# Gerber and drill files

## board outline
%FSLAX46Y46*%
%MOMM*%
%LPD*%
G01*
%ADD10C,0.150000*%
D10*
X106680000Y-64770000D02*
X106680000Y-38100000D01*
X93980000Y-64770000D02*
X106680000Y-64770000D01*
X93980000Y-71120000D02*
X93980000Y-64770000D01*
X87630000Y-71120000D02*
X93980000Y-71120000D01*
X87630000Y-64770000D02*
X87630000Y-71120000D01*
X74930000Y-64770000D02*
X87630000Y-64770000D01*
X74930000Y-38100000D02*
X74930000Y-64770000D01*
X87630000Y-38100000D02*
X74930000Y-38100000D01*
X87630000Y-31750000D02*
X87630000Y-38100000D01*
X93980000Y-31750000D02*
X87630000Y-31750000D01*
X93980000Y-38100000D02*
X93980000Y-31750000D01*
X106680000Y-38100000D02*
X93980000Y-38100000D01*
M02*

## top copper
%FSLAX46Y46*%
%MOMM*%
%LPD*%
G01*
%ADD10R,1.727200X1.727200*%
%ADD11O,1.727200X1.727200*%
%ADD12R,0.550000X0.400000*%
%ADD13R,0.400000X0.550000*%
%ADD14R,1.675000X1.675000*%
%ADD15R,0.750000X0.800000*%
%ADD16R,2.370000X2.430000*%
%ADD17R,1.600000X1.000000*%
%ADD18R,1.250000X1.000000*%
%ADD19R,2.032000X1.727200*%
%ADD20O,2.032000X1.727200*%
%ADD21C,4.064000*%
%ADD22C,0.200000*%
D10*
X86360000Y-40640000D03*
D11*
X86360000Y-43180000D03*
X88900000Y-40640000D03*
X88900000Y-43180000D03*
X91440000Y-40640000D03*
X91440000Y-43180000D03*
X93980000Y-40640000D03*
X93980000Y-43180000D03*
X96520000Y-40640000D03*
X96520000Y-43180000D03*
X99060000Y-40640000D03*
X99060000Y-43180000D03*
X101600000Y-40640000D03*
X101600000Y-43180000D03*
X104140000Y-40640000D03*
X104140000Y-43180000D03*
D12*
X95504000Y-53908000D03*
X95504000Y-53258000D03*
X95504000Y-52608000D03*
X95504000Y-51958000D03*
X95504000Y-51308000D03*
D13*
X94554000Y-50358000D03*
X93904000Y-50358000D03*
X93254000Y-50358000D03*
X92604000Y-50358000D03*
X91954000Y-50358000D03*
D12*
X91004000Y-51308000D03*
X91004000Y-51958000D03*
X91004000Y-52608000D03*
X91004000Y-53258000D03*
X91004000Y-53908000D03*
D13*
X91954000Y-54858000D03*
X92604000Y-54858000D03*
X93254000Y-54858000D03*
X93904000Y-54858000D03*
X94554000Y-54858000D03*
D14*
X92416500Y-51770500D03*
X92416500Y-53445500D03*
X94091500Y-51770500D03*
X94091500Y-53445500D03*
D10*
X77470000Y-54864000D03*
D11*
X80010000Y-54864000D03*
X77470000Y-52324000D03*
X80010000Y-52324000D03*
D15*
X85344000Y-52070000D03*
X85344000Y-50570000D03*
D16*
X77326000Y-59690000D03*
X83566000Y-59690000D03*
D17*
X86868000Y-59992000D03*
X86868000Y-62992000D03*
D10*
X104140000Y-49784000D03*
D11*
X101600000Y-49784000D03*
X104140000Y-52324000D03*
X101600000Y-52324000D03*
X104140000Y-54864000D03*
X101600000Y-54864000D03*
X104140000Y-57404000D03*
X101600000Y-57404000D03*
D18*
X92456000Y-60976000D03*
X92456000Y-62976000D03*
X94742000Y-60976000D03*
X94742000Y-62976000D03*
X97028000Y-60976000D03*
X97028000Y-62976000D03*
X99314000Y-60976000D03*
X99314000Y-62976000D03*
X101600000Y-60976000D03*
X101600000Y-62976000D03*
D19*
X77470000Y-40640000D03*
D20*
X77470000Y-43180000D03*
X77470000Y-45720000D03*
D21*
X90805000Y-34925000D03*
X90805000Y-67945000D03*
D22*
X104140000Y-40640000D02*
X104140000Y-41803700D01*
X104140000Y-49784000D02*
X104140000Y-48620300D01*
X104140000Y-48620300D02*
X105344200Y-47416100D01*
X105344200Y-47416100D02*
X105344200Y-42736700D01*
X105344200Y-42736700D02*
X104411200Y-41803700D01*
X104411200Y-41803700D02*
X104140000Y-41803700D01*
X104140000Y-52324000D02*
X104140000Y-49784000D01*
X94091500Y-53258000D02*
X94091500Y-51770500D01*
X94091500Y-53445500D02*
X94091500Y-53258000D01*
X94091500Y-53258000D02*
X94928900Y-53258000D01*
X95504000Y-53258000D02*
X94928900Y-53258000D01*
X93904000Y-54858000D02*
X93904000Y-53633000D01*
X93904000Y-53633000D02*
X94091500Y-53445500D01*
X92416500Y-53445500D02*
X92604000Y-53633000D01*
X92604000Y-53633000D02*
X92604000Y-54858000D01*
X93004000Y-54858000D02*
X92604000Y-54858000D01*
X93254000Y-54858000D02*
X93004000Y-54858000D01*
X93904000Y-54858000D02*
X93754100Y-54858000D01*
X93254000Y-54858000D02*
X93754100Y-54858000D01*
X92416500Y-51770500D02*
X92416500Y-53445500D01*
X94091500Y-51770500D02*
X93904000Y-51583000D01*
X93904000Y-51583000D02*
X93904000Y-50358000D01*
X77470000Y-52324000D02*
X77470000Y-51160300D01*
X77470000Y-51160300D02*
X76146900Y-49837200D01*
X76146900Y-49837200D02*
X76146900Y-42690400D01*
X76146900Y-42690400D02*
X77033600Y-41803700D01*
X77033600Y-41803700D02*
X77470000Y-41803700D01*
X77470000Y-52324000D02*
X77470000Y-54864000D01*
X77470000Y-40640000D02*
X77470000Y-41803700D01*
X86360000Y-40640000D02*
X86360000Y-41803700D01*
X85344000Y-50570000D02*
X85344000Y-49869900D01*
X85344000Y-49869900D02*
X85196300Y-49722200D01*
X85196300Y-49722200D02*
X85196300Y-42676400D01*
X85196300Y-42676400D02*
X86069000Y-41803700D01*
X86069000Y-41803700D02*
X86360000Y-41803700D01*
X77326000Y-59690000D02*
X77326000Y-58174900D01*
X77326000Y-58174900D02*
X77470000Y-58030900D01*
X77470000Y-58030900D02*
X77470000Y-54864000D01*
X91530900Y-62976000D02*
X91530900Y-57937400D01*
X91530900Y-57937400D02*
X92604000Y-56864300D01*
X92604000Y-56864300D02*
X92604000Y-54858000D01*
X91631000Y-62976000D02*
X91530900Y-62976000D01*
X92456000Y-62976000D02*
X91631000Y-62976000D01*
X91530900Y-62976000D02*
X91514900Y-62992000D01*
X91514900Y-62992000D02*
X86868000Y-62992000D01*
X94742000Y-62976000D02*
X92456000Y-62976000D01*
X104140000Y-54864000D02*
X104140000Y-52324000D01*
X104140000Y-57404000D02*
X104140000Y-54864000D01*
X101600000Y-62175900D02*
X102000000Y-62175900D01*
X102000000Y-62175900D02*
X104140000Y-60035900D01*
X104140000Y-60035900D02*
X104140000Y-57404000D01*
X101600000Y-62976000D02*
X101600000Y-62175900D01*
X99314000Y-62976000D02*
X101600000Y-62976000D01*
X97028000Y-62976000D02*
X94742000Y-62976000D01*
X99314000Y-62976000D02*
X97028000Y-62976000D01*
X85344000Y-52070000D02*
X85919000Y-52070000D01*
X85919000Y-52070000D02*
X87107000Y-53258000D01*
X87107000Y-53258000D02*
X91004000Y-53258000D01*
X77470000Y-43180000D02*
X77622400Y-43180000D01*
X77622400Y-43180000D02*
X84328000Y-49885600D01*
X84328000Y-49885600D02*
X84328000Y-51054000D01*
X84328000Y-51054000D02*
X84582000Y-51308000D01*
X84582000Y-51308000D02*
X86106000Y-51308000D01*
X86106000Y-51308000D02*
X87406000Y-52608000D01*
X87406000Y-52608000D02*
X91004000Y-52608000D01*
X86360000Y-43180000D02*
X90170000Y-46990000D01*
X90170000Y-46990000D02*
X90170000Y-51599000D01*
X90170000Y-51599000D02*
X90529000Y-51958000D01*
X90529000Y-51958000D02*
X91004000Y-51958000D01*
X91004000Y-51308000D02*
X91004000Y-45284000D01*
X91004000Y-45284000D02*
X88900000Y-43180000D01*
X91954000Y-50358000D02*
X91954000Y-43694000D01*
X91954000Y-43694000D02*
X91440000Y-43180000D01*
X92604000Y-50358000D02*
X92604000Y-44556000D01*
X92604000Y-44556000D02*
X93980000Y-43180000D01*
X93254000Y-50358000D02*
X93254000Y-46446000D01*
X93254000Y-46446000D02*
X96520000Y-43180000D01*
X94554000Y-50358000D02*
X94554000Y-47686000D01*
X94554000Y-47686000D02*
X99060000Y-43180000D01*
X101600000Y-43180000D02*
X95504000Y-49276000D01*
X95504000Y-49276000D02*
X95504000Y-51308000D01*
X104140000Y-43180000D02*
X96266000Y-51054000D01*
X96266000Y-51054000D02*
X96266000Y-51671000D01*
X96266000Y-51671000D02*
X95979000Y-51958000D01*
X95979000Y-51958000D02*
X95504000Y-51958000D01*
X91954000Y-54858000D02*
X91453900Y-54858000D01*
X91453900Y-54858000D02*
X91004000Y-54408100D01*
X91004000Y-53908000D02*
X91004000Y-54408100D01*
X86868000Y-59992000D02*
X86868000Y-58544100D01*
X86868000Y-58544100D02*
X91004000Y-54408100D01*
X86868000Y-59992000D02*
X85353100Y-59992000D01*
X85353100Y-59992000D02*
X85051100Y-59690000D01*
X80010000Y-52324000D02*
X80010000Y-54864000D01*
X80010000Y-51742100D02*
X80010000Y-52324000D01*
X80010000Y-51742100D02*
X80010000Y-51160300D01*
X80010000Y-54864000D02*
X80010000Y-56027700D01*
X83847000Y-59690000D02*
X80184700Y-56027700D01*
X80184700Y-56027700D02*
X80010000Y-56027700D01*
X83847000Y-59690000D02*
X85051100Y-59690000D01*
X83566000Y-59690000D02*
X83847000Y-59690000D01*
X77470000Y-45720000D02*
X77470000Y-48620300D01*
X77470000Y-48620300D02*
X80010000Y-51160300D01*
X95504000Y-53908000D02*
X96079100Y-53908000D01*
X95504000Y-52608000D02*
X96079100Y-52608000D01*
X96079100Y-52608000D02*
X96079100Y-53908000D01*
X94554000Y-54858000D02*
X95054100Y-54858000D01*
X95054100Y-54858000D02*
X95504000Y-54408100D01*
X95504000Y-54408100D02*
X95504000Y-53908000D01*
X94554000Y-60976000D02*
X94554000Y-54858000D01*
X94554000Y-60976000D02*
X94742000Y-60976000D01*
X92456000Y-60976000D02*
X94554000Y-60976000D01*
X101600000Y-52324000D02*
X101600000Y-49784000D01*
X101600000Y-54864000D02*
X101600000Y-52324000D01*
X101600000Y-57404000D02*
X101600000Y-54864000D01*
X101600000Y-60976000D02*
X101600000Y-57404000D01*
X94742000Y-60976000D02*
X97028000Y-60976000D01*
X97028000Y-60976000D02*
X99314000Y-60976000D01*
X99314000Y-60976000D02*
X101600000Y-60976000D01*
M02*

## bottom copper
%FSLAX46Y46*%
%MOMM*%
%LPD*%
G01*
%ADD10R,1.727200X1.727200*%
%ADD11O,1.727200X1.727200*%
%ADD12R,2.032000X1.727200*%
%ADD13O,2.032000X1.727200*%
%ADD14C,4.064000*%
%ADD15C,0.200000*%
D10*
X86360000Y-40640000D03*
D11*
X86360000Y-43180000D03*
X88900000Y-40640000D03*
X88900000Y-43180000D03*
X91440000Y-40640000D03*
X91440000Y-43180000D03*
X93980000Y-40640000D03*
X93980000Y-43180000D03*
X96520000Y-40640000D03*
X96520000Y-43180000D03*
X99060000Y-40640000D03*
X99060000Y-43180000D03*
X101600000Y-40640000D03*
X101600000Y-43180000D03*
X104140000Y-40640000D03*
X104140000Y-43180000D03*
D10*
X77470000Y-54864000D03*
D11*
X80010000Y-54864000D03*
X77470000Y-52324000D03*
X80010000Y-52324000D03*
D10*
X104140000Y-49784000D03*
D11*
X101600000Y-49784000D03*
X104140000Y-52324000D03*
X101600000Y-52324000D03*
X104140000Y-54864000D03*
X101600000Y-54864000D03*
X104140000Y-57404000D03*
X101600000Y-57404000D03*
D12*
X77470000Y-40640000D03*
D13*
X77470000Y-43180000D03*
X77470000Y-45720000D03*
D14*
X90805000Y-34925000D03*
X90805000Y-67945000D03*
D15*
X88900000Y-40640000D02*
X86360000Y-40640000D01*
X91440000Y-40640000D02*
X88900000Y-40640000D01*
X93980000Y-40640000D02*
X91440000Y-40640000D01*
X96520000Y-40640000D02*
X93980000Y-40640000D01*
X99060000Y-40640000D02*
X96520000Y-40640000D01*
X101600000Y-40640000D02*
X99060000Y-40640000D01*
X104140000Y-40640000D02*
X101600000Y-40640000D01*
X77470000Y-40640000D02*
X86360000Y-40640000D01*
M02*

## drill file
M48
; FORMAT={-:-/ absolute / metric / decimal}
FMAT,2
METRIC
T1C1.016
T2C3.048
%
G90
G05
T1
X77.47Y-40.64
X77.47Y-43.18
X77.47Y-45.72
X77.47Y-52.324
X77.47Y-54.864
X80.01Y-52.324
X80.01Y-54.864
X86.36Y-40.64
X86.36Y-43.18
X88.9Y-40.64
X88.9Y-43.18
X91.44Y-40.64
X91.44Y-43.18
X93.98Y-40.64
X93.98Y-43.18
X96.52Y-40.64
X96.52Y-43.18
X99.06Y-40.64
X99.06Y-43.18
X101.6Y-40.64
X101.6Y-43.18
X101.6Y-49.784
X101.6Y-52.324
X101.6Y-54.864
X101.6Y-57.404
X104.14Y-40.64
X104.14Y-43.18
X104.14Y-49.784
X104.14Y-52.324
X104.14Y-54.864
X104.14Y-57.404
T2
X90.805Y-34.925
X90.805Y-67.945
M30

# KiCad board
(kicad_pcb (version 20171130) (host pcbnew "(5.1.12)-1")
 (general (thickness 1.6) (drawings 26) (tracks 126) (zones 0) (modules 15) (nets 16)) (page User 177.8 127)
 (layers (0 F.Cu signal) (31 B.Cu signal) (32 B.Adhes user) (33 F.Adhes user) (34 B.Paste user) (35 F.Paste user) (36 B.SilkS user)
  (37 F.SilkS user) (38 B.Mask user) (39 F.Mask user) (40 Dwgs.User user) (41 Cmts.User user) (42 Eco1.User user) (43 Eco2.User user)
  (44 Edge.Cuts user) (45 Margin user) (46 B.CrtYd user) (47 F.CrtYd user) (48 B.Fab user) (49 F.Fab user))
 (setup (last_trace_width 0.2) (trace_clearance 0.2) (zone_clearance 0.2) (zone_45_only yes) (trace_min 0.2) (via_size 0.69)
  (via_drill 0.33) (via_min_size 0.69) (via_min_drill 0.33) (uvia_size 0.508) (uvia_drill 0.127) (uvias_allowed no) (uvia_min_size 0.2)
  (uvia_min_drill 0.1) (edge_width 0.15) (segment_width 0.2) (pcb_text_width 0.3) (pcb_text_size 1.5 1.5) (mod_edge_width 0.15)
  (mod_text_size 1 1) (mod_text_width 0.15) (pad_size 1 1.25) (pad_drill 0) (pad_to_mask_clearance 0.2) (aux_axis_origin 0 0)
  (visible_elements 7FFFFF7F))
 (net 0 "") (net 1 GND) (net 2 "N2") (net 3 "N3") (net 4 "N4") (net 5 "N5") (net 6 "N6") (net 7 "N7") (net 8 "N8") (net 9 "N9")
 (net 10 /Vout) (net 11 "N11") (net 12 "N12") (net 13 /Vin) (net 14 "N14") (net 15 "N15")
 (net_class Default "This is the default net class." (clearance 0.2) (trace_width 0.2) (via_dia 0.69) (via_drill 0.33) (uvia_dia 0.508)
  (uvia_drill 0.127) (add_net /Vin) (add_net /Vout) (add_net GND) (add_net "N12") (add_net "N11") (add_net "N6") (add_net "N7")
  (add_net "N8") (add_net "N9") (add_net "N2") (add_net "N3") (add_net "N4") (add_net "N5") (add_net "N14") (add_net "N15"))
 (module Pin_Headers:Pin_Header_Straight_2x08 (layer B.Cu) (at 86.36 40.64 270)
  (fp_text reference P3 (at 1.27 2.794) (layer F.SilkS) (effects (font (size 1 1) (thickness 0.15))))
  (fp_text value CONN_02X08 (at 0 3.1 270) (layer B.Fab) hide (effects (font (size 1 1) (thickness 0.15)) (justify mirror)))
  (pad 1 thru_hole rect (at 0 0 270) (size 1.7272 1.7272) (drill 1.016) (layers *.Cu *.Mask B.SilkS) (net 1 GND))
  (pad 2 thru_hole oval (at 2.54 0 270) (size 1.7272 1.7272) (drill 1.016) (layers *.Cu *.Mask B.SilkS) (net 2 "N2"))
  (pad 3 thru_hole oval (at 0 -2.54 270) (size 1.7272 1.7272) (drill 1.016) (layers *.Cu *.Mask B.SilkS) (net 1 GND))
  (pad 4 thru_hole oval (at 2.54 -2.54 270) (size 1.7272 1.7272) (drill 1.016) (layers *.Cu *.Mask B.SilkS) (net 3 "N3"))
  (pad 5 thru_hole oval (at 0 -5.08 270) (size 1.7272 1.7272) (drill 1.016) (layers *.Cu *.Mask B.SilkS) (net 1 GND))
  (pad 6 thru_hole oval (at 2.54 -5.08 270) (size 1.7272 1.7272) (drill 1.016) (layers *.Cu *.Mask B.SilkS) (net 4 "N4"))
  (pad 7 thru_hole oval (at 0 -7.62 270) (size 1.7272 1.7272) (drill 1.016) (layers *.Cu *.Mask B.SilkS) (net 1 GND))
  (pad 8 thru_hole oval (at 2.54 -7.62 270) (size 1.7272 1.7272) (drill 1.016) (layers *.Cu *.Mask B.SilkS) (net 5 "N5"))
  (pad 9 thru_hole oval (at 0 -10.16 270) (size 1.7272 1.7272) (drill 1.016) (layers *.Cu *.Mask B.SilkS) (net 1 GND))
  (pad 10 thru_hole oval (at 2.54 -10.16 270) (size 1.7272 1.7272) (drill 1.016) (layers *.Cu *.Mask B.SilkS) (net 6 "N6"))
  (pad 11 thru_hole oval (at 0 -12.7 270) (size 1.7272 1.7272) (drill 1.016) (layers *.Cu *.Mask B.SilkS) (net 1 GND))
  (pad 12 thru_hole oval (at 2.54 -12.7 270) (size 1.7272 1.7272) (drill 1.016) (layers *.Cu *.Mask B.SilkS) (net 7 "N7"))
  (pad 13 thru_hole oval (at 0 -15.24 270) (size 1.7272 1.7272) (drill 1.016) (layers *.Cu *.Mask B.SilkS) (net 1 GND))
  (pad 14 thru_hole oval (at 2.54 -15.24 270) (size 1.7272 1.7272) (drill 1.016) (layers *.Cu *.Mask B.SilkS) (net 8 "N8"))
  (pad 15 thru_hole oval (at 0 -17.78 270) (size 1.7272 1.7272) (drill 1.016) (layers *.Cu *.Mask B.SilkS) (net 1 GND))
  (pad 16 thru_hole oval (at 2.54 -17.78 270) (size 1.7272 1.7272) (drill 1.016) (layers *.Cu *.Mask B.SilkS) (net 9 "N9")))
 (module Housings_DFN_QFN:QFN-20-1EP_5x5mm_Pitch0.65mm (layer F.Cu) (at 93.254 52.608 180)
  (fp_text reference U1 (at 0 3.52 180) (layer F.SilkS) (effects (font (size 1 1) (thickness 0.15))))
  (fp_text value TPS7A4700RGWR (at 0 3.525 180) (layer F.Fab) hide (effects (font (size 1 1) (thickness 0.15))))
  (pad 1 smd rect (at -2.25 -1.3 180) (size 0.55 0.4) (layers F.Cu F.Paste F.Mask) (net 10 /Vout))
  (pad 2 smd rect (at -2.25 -0.65 180) (size 0.55 0.4) (layers F.Cu F.Paste F.Mask) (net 1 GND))
  (pad 3 smd rect (at -2.25 0 180) (size 0.55 0.4) (layers F.Cu F.Paste F.Mask) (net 10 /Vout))
  (pad 4 smd rect (at -2.25 0.65 180) (size 0.55 0.4) (layers F.Cu F.Paste F.Mask) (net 9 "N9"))
  (pad 5 smd rect (at -2.25 1.3 180) (size 0.55 0.4) (layers F.Cu F.Paste F.Mask) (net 8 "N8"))
  (pad 6 smd rect (at -1.3 2.25 270) (size 0.55 0.4) (layers F.Cu F.Paste F.Mask) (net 7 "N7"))
  (pad 7 smd rect (at -0.65 2.25 270) (size 0.55 0.4) (layers F.Cu F.Paste F.Mask) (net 1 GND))
  (pad 8 smd rect (at 0 2.25 270) (size 0.55 0.4) (layers F.Cu F.Paste F.Mask) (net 6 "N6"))
  (pad 9 smd rect (at 0.65 2.25 270) (size 0.55 0.4) (layers F.Cu F.Paste F.Mask) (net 5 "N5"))
  (pad 10 smd rect (at 1.3 2.25 270) (size 0.55 0.4) (layers F.Cu F.Paste F.Mask) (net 4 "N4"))
  (pad 11 smd rect (at 2.25 1.3 180) (size 0.55 0.4) (layers F.Cu F.Paste F.Mask) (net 3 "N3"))
  (pad 12 smd rect (at 2.25 0.65 180) (size 0.55 0.4) (layers F.Cu F.Paste F.Mask) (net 2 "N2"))
  (pad 13 smd rect (at 2.25 0 180) (size 0.55 0.4) (layers F.Cu F.Paste F.Mask) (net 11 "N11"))
  (pad 14 smd rect (at 2.25 -0.65 180) (size 0.55 0.4) (layers F.Cu F.Paste F.Mask) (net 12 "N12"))
  (pad 15 smd rect (at 2.25 -1.3 180) (size 0.55 0.4) (layers F.Cu F.Paste F.Mask) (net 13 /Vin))
  (pad 16 smd rect (at 1.3 -2.25 270) (size 0.55 0.4) (layers F.Cu F.Paste F.Mask) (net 13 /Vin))
  (pad 17 smd rect (at 0.65 -2.25 270) (size 0.55 0.4) (layers F.Cu F.Paste F.Mask) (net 1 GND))
  (pad 18 smd rect (at 0 -2.25 270) (size 0.55 0.4) (layers F.Cu F.Paste F.Mask) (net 1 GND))
  (pad 19 smd rect (at -0.65 -2.25 270) (size 0.55 0.4) (layers F.Cu F.Paste F.Mask) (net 1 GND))
  (pad 20 smd rect (at -1.3 -2.25 270) (size 0.55 0.4) (layers F.Cu F.Paste F.Mask) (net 10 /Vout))
  (pad 21 smd rect (at 0.8375 0.8375 180) (size 1.675 1.675) (layers F.Cu F.Paste F.Mask) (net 1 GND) (solder_paste_margin_ratio -0.2))
  (pad 21 smd rect (at 0.8375 -0.8375 180) (size 1.675 1.675) (layers F.Cu F.Paste F.Mask) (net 1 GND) (solder_paste_margin_ratio -0.2))
  (pad 21 smd rect (at -0.8375 0.8375 180) (size 1.675 1.675) (layers F.Cu F.Paste F.Mask) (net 1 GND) (solder_paste_margin_ratio -0.2))
  (pad 21 smd rect (at -0.8375 -0.8375 180) (size 1.675 1.675) (layers F.Cu F.Paste F.Mask) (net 1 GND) (solder_paste_margin_ratio -0.2)))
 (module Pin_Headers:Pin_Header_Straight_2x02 (layer B.Cu) (at 77.47 54.864)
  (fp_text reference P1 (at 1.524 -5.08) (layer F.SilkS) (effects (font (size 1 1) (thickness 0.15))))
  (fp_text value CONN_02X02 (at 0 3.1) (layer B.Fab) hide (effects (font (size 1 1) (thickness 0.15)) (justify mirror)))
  (pad 1 thru_hole rect (at 0 0) (size 1.7272 1.7272) (drill 1.016) (layers *.Cu *.Mask B.SilkS) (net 1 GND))
  (pad 2 thru_hole oval (at 2.54 0) (size 1.7272 1.7272) (drill 1.016) (layers *.Cu *.Mask B.SilkS) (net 13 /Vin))
  (pad 3 thru_hole oval (at 0 -2.54) (size 1.7272 1.7272) (drill 1.016) (layers *.Cu *.Mask B.SilkS) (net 1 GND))
  (pad 4 thru_hole oval (at 2.54 -2.54) (size 1.7272 1.7272) (drill 1.016) (layers *.Cu *.Mask B.SilkS) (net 13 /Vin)))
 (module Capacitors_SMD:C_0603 (layer F.Cu) (at 85.344 51.32 90)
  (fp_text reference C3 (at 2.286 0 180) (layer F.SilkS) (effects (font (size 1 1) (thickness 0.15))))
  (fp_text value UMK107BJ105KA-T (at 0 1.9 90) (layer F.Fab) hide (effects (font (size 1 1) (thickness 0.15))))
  (pad 1 smd rect (at -0.75 0 90) (size 0.8 0.75) (layers F.Cu F.Paste F.Mask) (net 12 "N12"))
  (pad 2 smd rect (at 0.75 0 90) (size 0.8 0.75) (layers F.Cu F.Paste F.Mask) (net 1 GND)))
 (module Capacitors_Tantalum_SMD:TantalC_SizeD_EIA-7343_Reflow (layer F.Cu) (at 80.446 59.69 180)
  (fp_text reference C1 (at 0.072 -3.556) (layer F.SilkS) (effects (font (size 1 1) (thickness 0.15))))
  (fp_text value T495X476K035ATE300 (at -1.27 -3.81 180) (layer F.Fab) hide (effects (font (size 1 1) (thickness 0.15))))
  (pad 2 smd rect (at 3.12 0 180) (size 2.37 2.43) (layers F.Cu F.Paste F.Mask) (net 1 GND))
  (pad 1 smd rect (at -3.12 0 180) (size 2.37 2.43) (layers F.Cu F.Paste F.Mask) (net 13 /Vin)))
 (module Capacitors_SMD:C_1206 (layer F.Cu) (at 86.868 61.492 270)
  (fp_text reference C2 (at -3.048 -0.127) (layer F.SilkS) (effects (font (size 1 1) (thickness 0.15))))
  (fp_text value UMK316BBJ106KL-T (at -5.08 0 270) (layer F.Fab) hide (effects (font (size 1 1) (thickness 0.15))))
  (pad 1 smd rect (at -1.5 0 270) (size 1 1.6) (layers F.Cu F.Paste F.Mask) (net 13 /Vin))
  (pad 2 smd rect (at 1.5 0 270) (size 1 1.6) (layers F.Cu F.Paste F.Mask) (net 1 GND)))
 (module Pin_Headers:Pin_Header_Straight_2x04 (layer B.Cu) (at 104.14 49.784 180)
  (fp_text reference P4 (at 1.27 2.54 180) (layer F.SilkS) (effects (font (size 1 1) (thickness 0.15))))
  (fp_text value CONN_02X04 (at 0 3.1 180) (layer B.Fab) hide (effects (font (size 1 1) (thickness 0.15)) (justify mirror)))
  (pad 1 thru_hole rect (at 0 0 180) (size 1.7272 1.7272) (drill 1.016) (layers *.Cu *.Mask B.SilkS) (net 1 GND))
  (pad 2 thru_hole oval (at 2.54 0 180) (size 1.7272 1.7272) (drill 1.016) (layers *.Cu *.Mask B.SilkS) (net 10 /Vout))
  (pad 3 thru_hole oval (at 0 -2.54 180) (size 1.7272 1.7272) (drill 1.016) (layers *.Cu *.Mask B.SilkS) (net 1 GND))
  (pad 4 thru_hole oval (at 2.54 -2.54 180) (size 1.7272 1.7272) (drill 1.016) (layers *.Cu *.Mask B.SilkS) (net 10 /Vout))
  (pad 5 thru_hole oval (at 0 -5.08 180) (size 1.7272 1.7272) (drill 1.016) (layers *.Cu *.Mask B.SilkS) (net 1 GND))
  (pad 6 thru_hole oval (at 2.54 -5.08 180) (size 1.7272 1.7272) (drill 1.016) (layers *.Cu *.Mask B.SilkS) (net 10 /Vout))
  (pad 7 thru_hole oval (at 0 -7.62 180) (size 1.7272 1.7272) (drill 1.016) (layers *.Cu *.Mask B.SilkS) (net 1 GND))
  (pad 8 thru_hole oval (at 2.54 -7.62 180) (size 1.7272 1.7272) (drill 1.016) (layers *.Cu *.Mask B.SilkS) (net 10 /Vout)))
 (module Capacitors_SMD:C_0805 (layer F.Cu) (at 92.456 61.976 270)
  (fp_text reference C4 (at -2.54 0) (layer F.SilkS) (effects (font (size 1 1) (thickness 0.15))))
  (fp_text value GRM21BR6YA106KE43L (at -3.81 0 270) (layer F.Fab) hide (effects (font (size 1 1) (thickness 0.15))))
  (pad 1 smd rect (at -1 0 270) (size 1 1.25) (layers F.Cu F.Paste F.Mask) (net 10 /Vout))
  (pad 2 smd rect (at 1 0 270) (size 1 1.25) (layers F.Cu F.Paste F.Mask) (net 1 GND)))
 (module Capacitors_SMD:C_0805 (layer F.Cu) (at 94.742 61.976 270)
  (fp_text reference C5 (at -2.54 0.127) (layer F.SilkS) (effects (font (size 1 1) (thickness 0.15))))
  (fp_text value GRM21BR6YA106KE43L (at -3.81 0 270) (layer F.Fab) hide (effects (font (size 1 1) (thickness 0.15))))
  (pad 1 smd rect (at -1 0 270) (size 1 1.25) (layers F.Cu F.Paste F.Mask) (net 10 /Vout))
  (pad 2 smd rect (at 1 0 270) (size 1 1.25) (layers F.Cu F.Paste F.Mask) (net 1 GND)))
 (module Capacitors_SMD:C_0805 (layer F.Cu) (at 97.028 61.976 270)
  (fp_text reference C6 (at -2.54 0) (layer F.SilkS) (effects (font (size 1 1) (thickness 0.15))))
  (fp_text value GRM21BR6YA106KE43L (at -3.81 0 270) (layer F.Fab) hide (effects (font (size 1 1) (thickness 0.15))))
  (pad 1 smd rect (at -1 0 270) (size 1 1.25) (layers F.Cu F.Paste F.Mask) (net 10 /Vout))
  (pad 2 smd rect (at 1 0 270) (size 1 1.25) (layers F.Cu F.Paste F.Mask) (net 1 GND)))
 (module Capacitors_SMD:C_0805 (layer F.Cu) (at 99.314 61.976 270)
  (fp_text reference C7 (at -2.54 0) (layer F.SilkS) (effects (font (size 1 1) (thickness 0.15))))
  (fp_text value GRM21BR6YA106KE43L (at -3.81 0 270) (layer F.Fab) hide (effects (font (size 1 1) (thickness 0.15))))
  (pad 1 smd rect (at -1 0 270) (size 1 1.25) (layers F.Cu F.Paste F.Mask) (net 10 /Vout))
  (pad 2 smd rect (at 1 0 270) (size 1 1.25) (layers F.Cu F.Paste F.Mask) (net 1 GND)))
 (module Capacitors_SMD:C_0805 (layer F.Cu) (at 101.6 61.976 270)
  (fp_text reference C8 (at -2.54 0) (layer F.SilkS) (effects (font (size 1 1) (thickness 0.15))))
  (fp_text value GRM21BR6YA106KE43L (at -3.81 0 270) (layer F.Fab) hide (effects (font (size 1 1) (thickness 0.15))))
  (pad 1 smd rect (at -1 0 270) (size 1 1.25) (layers F.Cu F.Paste F.Mask) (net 10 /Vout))
  (pad 2 smd rect (at 1 0 270) (size 1 1.25) (layers F.Cu F.Paste F.Mask) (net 1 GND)))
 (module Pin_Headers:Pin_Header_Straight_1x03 (layer B.Cu) (at 77.47 40.64 180)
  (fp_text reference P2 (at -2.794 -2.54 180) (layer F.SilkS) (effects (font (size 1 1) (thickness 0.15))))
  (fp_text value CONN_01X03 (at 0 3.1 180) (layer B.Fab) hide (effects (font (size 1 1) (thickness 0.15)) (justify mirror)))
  (pad 1 thru_hole rect (at 0 0 180) (size 2.032 1.7272) (drill 1.016) (layers *.Cu *.Mask B.SilkS) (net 1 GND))
  (pad 2 thru_hole oval (at 0 -2.54 180) (size 2.032 1.7272) (drill 1.016) (layers *.Cu *.Mask B.SilkS) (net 11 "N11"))
  (pad 3 thru_hole oval (at 0 -5.08 180) (size 2.032 1.7272) (drill 1.016) (layers *.Cu *.Mask B.SilkS) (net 13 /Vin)))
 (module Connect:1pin (layer F.Cu) (at 90.805 34.925)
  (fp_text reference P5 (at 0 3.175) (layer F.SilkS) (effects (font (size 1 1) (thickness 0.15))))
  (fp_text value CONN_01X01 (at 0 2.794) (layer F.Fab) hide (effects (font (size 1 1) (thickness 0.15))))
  (pad 1 thru_hole circle (at 0 0) (size 4.064 4.064) (drill 3.048) (layers *.Cu *.Mask F.SilkS) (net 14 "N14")))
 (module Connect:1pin (layer F.Cu) (at 90.805 67.945)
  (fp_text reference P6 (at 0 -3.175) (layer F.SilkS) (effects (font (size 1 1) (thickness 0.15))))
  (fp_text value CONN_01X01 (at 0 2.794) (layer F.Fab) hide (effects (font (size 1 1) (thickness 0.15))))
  (pad 1 thru_hole circle (at 0 0) (size 4.064 4.064) (drill 3.048) (layers *.Cu *.Mask F.SilkS) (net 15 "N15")))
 (gr_line (start 106.68 64.77) (end 106.68 38.1) (layer Edge.Cuts) (width 0.15))
 (gr_line (start 93.98 64.77) (end 106.68 64.77) (layer Edge.Cuts) (width 0.15))
 (gr_line (start 93.98 71.12) (end 93.98 64.77) (layer Edge.Cuts) (width 0.15))
 (gr_line (start 87.63 71.12) (end 93.98 71.12) (layer Edge.Cuts) (width 0.15))
 (gr_line (start 87.63 64.77) (end 87.63 71.12) (layer Edge.Cuts) (width 0.15))
 (gr_line (start 74.93 64.77) (end 87.63 64.77) (layer Edge.Cuts) (width 0.15))
 (gr_line (start 74.93 38.1) (end 74.93 64.77) (layer Edge.Cuts) (width 0.15))
 (gr_line (start 87.63 38.1) (end 74.93 38.1) (layer Edge.Cuts) (width 0.15))
 (gr_line (start 87.63 31.75) (end 87.63 38.1) (layer Edge.Cuts) (width 0.15))
 (gr_line (start 93.98 31.75) (end 87.63 31.75) (layer Edge.Cuts) (width 0.15))
 (gr_line (start 93.98 38.1) (end 93.98 31.75) (layer Edge.Cuts) (width 0.15))
 (gr_line (start 106.68 38.1) (end 93.98 38.1) (layer Edge.Cuts) (width 0.15))
 (segment (start 88.9 40.64) (end 86.36 40.64) (width 0.2) (layer B.Cu) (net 1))
 (segment (start 91.44 40.64) (end 88.9 40.64) (width 0.2) (layer B.Cu) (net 1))
 (segment (start 93.98 40.64) (end 91.44 40.64) (width 0.2) (layer B.Cu) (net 1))
 (segment (start 96.52 40.64) (end 93.98 40.64) (width 0.2) (layer B.Cu) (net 1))
 (segment (start 99.06 40.64) (end 96.52 40.64) (width 0.2) (layer B.Cu) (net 1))
 (segment (start 101.6 40.64) (end 99.06 40.64) (width 0.2) (layer B.Cu) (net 1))
 (segment (start 104.14 40.64) (end 101.6 40.64) (width 0.2) (layer B.Cu) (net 1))
 (segment (start 104.14 40.64) (end 104.14 41.8037) (width 0.2) (layer F.Cu) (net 1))
 (segment (start 104.14 49.784) (end 104.14 48.6203) (width 0.2) (layer F.Cu) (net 1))
 (segment (start 104.14 48.6203) (end 105.3442 47.4161) (width 0.2) (layer F.Cu) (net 1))
 (segment (start 105.3442 47.4161) (end 105.3442 42.7367) (width 0.2) (layer F.Cu) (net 1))
 (segment (start 105.3442 42.7367) (end 104.4112 41.8037) (width 0.2) (layer F.Cu) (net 1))
 (segment (start 104.4112 41.8037) (end 104.14 41.8037) (width 0.2) (layer F.Cu) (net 1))
 (segment (start 104.14 52.324) (end 104.14 49.784) (width 0.2) (layer F.Cu) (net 1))
 (segment (start 94.0915 53.258) (end 94.0915 51.7705) (width 0.2) (layer F.Cu) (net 1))
 (segment (start 94.0915 53.4455) (end 94.0915 53.258) (width 0.2) (layer F.Cu) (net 1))
 (segment (start 94.0915 53.258) (end 94.9289 53.258) (width 0.2) (layer F.Cu) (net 1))
 (segment (start 95.504 53.258) (end 94.9289 53.258) (width 0.2) (layer F.Cu) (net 1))
 (segment (start 93.904 54.858) (end 93.904 53.633) (width 0.2) (layer F.Cu) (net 1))
 (segment (start 93.904 53.633) (end 94.0915 53.4455) (width 0.2) (layer F.Cu) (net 1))
 (segment (start 92.4165 53.4455) (end 92.604 53.633) (width 0.2) (layer F.Cu) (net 1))
 (segment (start 92.604 53.633) (end 92.604 54.858) (width 0.2) (layer F.Cu) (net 1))
 (segment (start 93.004 54.858) (end 92.604 54.858) (width 0.2) (layer F.Cu) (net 1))
 (segment (start 93.254 54.858) (end 93.004 54.858) (width 0.2) (layer F.Cu) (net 1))
 (segment (start 93.904 54.858) (end 93.7541 54.858) (width 0.2) (layer F.Cu) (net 1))
 (segment (start 93.254 54.858) (end 93.7541 54.858) (width 0.2) (layer F.Cu) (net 1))
 (segment (start 92.4165 51.7705) (end 92.4165 53.4455) (width 0.2) (layer F.Cu) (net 1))
 (segment (start 94.0915 51.7705) (end 93.904 51.583) (width 0.2) (layer F.Cu) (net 1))
 (segment (start 93.904 51.583) (end 93.904 50.358) (width 0.2) (layer F.Cu) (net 1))
 (segment (start 77.47 52.324) (end 77.47 51.1603) (width 0.2) (layer F.Cu) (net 1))
 (segment (start 77.47 51.1603) (end 76.1469 49.8372) (width 0.2) (layer F.Cu) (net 1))
 (segment (start 76.1469 49.8372) (end 76.1469 42.6904) (width 0.2) (layer F.Cu) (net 1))
 (segment (start 76.1469 42.6904) (end 77.0336 41.8037) (width 0.2) (layer F.Cu) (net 1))
 (segment (start 77.0336 41.8037) (end 77.47 41.8037) (width 0.2) (layer F.Cu) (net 1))
 (segment (start 77.47 52.324) (end 77.47 54.864) (width 0.2) (layer F.Cu) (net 1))
 (segment (start 77.47 40.64) (end 77.47 41.8037) (width 0.2) (layer F.Cu) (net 1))
 (segment (start 86.36 40.64) (end 86.36 41.8037) (width 0.2) (layer F.Cu) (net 1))
 (segment (start 85.344 50.57) (end 85.344 49.8699) (width 0.2) (layer F.Cu) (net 1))
 (segment (start 85.344 49.8699) (end 85.1963 49.7222) (width 0.2) (layer F.Cu) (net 1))
 (segment (start 85.1963 49.7222) (end 85.1963 42.6764) (width 0.2) (layer F.Cu) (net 1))
 (segment (start 85.1963 42.6764) (end 86.069 41.8037) (width 0.2) (layer F.Cu) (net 1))
 (segment (start 86.069 41.8037) (end 86.36 41.8037) (width 0.2) (layer F.Cu) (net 1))
 (segment (start 77.326 59.69) (end 77.326 58.1749) (width 0.2) (layer F.Cu) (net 1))
 (segment (start 77.326 58.1749) (end 77.47 58.0309) (width 0.2) (layer F.Cu) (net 1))
 (segment (start 77.47 58.0309) (end 77.47 54.864) (width 0.2) (layer F.Cu) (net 1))
 (segment (start 91.5309 62.976) (end 91.5309 57.9374) (width 0.2) (layer F.Cu) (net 1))
 (segment (start 91.5309 57.9374) (end 92.604 56.8643) (width 0.2) (layer F.Cu) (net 1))
 (segment (start 92.604 56.8643) (end 92.604 54.858) (width 0.2) (layer F.Cu) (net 1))
 (segment (start 91.631 62.976) (end 91.5309 62.976) (width 0.2) (layer F.Cu) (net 1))
 (segment (start 92.456 62.976) (end 91.631 62.976) (width 0.2) (layer F.Cu) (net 1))
 (segment (start 91.5309 62.976) (end 91.5149 62.992) (width 0.2) (layer F.Cu) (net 1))
 (segment (start 91.5149 62.992) (end 86.868 62.992) (width 0.2) (layer F.Cu) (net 1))
 (segment (start 94.742 62.976) (end 92.456 62.976) (width 0.2) (layer F.Cu) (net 1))
 (segment (start 104.14 54.864) (end 104.14 52.324) (width 0.2) (layer F.Cu) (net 1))
 (segment (start 104.14 57.404) (end 104.14 54.864) (width 0.2) (layer F.Cu) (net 1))
 (segment (start 101.6 62.1759) (end 102 62.1759) (width 0.2) (layer F.Cu) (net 1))
 (segment (start 102 62.1759) (end 104.14 60.0359) (width 0.2) (layer F.Cu) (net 1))
 (segment (start 104.14 60.0359) (end 104.14 57.404) (width 0.2) (layer F.Cu) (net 1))
 (segment (start 101.6 62.976) (end 101.6 62.1759) (width 0.2) (layer F.Cu) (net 1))
 (segment (start 99.314 62.976) (end 101.6 62.976) (width 0.2) (layer F.Cu) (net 1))
 (segment (start 97.028 62.976) (end 94.742 62.976) (width 0.2) (layer F.Cu) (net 1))
 (segment (start 99.314 62.976) (end 97.028 62.976) (width 0.2) (layer F.Cu) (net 1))
 (segment (start 77.47 40.64) (end 86.36 40.64) (width 0.2) (layer B.Cu) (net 1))
 (segment (start 85.344 52.07) (end 85.919 52.07) (width 0.2) (layer F.Cu) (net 12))
 (segment (start 85.919 52.07) (end 87.107 53.258) (width 0.2) (layer F.Cu) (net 12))
 (segment (start 87.107 53.258) (end 91.004 53.258) (width 0.2) (layer F.Cu) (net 12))
 (segment (start 77.47 43.18) (end 77.6224 43.18) (width 0.2) (layer F.Cu) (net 11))
 (segment (start 77.6224 43.18) (end 84.328 49.8856) (width 0.2) (layer F.Cu) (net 11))
 (segment (start 84.328 49.8856) (end 84.328 51.054) (width 0.2) (layer F.Cu) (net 11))
 (segment (start 84.328 51.054) (end 84.582 51.308) (width 0.2) (layer F.Cu) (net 11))
 (segment (start 84.582 51.308) (end 86.106 51.308) (width 0.2) (layer F.Cu) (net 11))
 (segment (start 86.106 51.308) (end 87.406 52.608) (width 0.2) (layer F.Cu) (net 11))
 (segment (start 87.406 52.608) (end 91.004 52.608) (width 0.2) (layer F.Cu) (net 11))
 (segment (start 86.36 43.18) (end 90.17 46.99) (width 0.2) (layer F.Cu) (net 2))
 (segment (start 90.17 46.99) (end 90.17 51.599) (width 0.2) (layer F.Cu) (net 2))
 (segment (start 90.17 51.599) (end 90.529 51.958) (width 0.2) (layer F.Cu) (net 2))
 (segment (start 90.529 51.958) (end 91.004 51.958) (width 0.2) (layer F.Cu) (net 2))
 (segment (start 91.004 51.308) (end 91.004 45.284) (width 0.2) (layer F.Cu) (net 3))
 (segment (start 91.004 45.284) (end 88.9 43.18) (width 0.2) (layer F.Cu) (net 3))
 (segment (start 91.954 50.358) (end 91.954 43.694) (width 0.2) (layer F.Cu) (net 4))
 (segment (start 91.954 43.694) (end 91.44 43.18) (width 0.2) (layer F.Cu) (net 4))
 (segment (start 92.604 50.358) (end 92.604 44.556) (width 0.2) (layer F.Cu) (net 5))
 (segment (start 92.604 44.556) (end 93.98 43.18) (width 0.2) (layer F.Cu) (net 5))
 (segment (start 93.254 50.358) (end 93.254 46.446) (width 0.2) (layer F.Cu) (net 6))
 (segment (start 93.254 46.446) (end 96.52 43.18) (width 0.2) (layer F.Cu) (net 6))
 (segment (start 94.554 50.358) (end 94.554 47.686) (width 0.2) (layer F.Cu) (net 7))
 (segment (start 94.554 47.686) (end 99.06 43.18) (width 0.2) (layer F.Cu) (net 7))
 (segment (start 101.6 43.18) (end 95.504 49.276) (width 0.2) (layer F.Cu) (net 8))
 (segment (start 95.504 49.276) (end 95.504 51.308) (width 0.2) (layer F.Cu) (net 8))
 (segment (start 104.14 43.18) (end 96.266 51.054) (width 0.2) (layer F.Cu) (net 9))
 (segment (start 96.266 51.054) (end 96.266 51.671) (width 0.2) (layer F.Cu) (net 9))
 (segment (start 96.266 51.671) (end 95.979 51.958) (width 0.2) (layer F.Cu) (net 9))
 (segment (start 95.979 51.958) (end 95.504 51.958) (width 0.2) (layer F.Cu) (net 9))
 (segment (start 91.954 54.858) (end 91.4539 54.858) (width 0.2) (layer F.Cu) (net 13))
 (segment (start 91.4539 54.858) (end 91.004 54.4081) (width 0.2) (layer F.Cu) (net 13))
 (segment (start 91.004 53.908) (end 91.004 54.4081) (width 0.2) (layer F.Cu) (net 13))
 (segment (start 86.868 59.992) (end 86.868 58.5441) (width 0.2) (layer F.Cu) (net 13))
 (segment (start 86.868 58.5441) (end 91.004 54.4081) (width 0.2) (layer F.Cu) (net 13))
 (segment (start 86.868 59.992) (end 85.3531 59.992) (width 0.2) (layer F.Cu) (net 13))
 (segment (start 85.3531 59.992) (end 85.0511 59.69) (width 0.2) (layer F.Cu) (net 13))
 (segment (start 80.01 52.324) (end 80.01 54.864) (width 0.2) (layer F.Cu) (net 13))
 (segment (start 80.01 51.7421) (end 80.01 52.324) (width 0.2) (layer F.Cu) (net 13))
 (segment (start 80.01 51.7421) (end 80.01 51.1603) (width 0.2) (layer F.Cu) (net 13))
 (segment (start 80.01 54.864) (end 80.01 56.0277) (width 0.2) (layer F.Cu) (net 13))
 (segment (start 83.847 59.69) (end 80.1847 56.0277) (width 0.2) (layer F.Cu) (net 13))
 (segment (start 80.1847 56.0277) (end 80.01 56.0277) (width 0.2) (layer F.Cu) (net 13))
 (segment (start 83.847 59.69) (end 85.0511 59.69) (width 0.2) (layer F.Cu) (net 13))
 (segment (start 83.566 59.69) (end 83.847 59.69) (width 0.2) (layer F.Cu) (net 13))
 (segment (start 77.47 45.72) (end 77.47 48.6203) (width 0.2) (layer F.Cu) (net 13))
 (segment (start 77.47 48.6203) (end 80.01 51.1603) (width 0.2) (layer F.Cu) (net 13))
 (segment (start 95.504 53.908) (end 96.0791 53.908) (width 0.2) (layer F.Cu) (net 10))
 (segment (start 95.504 52.608) (end 96.0791 52.608) (width 0.2) (layer F.Cu) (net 10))
 (segment (start 96.0791 52.608) (end 96.0791 53.908) (width 0.2) (layer F.Cu) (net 10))
 (segment (start 94.554 54.858) (end 95.0541 54.858) (width 0.2) (layer F.Cu) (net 10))
 (segment (start 95.0541 54.858) (end 95.504 54.4081) (width 0.2) (layer F.Cu) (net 10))
 (segment (start 95.504 54.4081) (end 95.504 53.908) (width 0.2) (layer F.Cu) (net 10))
 (segment (start 94.554 60.976) (end 94.554 54.858) (width 0.2) (layer F.Cu) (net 10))
 (segment (start 94.554 60.976) (end 94.742 60.976) (width 0.2) (layer F.Cu) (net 10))
 (segment (start 92.456 60.976) (end 94.554 60.976) (width 0.2) (layer F.Cu) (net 10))
 (segment (start 101.6 52.324) (end 101.6 49.784) (width 0.2) (layer F.Cu) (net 10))
 (segment (start 101.6 54.864) (end 101.6 52.324) (width 0.2) (layer F.Cu) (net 10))
 (segment (start 101.6 57.404) (end 101.6 54.864) (width 0.2) (layer F.Cu) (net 10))
 (segment (start 101.6 60.976) (end 101.6 57.404) (width 0.2) (layer F.Cu) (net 10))
 (segment (start 94.742 60.976) (end 97.028 60.976) (width 0.2) (layer F.Cu) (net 10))
 (segment (start 97.028 60.976) (end 99.314 60.976) (width 0.2) (layer F.Cu) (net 10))
 (segment (start 99.314 60.976) (end 101.6 60.976) (width 0.2) (layer F.Cu) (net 10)))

